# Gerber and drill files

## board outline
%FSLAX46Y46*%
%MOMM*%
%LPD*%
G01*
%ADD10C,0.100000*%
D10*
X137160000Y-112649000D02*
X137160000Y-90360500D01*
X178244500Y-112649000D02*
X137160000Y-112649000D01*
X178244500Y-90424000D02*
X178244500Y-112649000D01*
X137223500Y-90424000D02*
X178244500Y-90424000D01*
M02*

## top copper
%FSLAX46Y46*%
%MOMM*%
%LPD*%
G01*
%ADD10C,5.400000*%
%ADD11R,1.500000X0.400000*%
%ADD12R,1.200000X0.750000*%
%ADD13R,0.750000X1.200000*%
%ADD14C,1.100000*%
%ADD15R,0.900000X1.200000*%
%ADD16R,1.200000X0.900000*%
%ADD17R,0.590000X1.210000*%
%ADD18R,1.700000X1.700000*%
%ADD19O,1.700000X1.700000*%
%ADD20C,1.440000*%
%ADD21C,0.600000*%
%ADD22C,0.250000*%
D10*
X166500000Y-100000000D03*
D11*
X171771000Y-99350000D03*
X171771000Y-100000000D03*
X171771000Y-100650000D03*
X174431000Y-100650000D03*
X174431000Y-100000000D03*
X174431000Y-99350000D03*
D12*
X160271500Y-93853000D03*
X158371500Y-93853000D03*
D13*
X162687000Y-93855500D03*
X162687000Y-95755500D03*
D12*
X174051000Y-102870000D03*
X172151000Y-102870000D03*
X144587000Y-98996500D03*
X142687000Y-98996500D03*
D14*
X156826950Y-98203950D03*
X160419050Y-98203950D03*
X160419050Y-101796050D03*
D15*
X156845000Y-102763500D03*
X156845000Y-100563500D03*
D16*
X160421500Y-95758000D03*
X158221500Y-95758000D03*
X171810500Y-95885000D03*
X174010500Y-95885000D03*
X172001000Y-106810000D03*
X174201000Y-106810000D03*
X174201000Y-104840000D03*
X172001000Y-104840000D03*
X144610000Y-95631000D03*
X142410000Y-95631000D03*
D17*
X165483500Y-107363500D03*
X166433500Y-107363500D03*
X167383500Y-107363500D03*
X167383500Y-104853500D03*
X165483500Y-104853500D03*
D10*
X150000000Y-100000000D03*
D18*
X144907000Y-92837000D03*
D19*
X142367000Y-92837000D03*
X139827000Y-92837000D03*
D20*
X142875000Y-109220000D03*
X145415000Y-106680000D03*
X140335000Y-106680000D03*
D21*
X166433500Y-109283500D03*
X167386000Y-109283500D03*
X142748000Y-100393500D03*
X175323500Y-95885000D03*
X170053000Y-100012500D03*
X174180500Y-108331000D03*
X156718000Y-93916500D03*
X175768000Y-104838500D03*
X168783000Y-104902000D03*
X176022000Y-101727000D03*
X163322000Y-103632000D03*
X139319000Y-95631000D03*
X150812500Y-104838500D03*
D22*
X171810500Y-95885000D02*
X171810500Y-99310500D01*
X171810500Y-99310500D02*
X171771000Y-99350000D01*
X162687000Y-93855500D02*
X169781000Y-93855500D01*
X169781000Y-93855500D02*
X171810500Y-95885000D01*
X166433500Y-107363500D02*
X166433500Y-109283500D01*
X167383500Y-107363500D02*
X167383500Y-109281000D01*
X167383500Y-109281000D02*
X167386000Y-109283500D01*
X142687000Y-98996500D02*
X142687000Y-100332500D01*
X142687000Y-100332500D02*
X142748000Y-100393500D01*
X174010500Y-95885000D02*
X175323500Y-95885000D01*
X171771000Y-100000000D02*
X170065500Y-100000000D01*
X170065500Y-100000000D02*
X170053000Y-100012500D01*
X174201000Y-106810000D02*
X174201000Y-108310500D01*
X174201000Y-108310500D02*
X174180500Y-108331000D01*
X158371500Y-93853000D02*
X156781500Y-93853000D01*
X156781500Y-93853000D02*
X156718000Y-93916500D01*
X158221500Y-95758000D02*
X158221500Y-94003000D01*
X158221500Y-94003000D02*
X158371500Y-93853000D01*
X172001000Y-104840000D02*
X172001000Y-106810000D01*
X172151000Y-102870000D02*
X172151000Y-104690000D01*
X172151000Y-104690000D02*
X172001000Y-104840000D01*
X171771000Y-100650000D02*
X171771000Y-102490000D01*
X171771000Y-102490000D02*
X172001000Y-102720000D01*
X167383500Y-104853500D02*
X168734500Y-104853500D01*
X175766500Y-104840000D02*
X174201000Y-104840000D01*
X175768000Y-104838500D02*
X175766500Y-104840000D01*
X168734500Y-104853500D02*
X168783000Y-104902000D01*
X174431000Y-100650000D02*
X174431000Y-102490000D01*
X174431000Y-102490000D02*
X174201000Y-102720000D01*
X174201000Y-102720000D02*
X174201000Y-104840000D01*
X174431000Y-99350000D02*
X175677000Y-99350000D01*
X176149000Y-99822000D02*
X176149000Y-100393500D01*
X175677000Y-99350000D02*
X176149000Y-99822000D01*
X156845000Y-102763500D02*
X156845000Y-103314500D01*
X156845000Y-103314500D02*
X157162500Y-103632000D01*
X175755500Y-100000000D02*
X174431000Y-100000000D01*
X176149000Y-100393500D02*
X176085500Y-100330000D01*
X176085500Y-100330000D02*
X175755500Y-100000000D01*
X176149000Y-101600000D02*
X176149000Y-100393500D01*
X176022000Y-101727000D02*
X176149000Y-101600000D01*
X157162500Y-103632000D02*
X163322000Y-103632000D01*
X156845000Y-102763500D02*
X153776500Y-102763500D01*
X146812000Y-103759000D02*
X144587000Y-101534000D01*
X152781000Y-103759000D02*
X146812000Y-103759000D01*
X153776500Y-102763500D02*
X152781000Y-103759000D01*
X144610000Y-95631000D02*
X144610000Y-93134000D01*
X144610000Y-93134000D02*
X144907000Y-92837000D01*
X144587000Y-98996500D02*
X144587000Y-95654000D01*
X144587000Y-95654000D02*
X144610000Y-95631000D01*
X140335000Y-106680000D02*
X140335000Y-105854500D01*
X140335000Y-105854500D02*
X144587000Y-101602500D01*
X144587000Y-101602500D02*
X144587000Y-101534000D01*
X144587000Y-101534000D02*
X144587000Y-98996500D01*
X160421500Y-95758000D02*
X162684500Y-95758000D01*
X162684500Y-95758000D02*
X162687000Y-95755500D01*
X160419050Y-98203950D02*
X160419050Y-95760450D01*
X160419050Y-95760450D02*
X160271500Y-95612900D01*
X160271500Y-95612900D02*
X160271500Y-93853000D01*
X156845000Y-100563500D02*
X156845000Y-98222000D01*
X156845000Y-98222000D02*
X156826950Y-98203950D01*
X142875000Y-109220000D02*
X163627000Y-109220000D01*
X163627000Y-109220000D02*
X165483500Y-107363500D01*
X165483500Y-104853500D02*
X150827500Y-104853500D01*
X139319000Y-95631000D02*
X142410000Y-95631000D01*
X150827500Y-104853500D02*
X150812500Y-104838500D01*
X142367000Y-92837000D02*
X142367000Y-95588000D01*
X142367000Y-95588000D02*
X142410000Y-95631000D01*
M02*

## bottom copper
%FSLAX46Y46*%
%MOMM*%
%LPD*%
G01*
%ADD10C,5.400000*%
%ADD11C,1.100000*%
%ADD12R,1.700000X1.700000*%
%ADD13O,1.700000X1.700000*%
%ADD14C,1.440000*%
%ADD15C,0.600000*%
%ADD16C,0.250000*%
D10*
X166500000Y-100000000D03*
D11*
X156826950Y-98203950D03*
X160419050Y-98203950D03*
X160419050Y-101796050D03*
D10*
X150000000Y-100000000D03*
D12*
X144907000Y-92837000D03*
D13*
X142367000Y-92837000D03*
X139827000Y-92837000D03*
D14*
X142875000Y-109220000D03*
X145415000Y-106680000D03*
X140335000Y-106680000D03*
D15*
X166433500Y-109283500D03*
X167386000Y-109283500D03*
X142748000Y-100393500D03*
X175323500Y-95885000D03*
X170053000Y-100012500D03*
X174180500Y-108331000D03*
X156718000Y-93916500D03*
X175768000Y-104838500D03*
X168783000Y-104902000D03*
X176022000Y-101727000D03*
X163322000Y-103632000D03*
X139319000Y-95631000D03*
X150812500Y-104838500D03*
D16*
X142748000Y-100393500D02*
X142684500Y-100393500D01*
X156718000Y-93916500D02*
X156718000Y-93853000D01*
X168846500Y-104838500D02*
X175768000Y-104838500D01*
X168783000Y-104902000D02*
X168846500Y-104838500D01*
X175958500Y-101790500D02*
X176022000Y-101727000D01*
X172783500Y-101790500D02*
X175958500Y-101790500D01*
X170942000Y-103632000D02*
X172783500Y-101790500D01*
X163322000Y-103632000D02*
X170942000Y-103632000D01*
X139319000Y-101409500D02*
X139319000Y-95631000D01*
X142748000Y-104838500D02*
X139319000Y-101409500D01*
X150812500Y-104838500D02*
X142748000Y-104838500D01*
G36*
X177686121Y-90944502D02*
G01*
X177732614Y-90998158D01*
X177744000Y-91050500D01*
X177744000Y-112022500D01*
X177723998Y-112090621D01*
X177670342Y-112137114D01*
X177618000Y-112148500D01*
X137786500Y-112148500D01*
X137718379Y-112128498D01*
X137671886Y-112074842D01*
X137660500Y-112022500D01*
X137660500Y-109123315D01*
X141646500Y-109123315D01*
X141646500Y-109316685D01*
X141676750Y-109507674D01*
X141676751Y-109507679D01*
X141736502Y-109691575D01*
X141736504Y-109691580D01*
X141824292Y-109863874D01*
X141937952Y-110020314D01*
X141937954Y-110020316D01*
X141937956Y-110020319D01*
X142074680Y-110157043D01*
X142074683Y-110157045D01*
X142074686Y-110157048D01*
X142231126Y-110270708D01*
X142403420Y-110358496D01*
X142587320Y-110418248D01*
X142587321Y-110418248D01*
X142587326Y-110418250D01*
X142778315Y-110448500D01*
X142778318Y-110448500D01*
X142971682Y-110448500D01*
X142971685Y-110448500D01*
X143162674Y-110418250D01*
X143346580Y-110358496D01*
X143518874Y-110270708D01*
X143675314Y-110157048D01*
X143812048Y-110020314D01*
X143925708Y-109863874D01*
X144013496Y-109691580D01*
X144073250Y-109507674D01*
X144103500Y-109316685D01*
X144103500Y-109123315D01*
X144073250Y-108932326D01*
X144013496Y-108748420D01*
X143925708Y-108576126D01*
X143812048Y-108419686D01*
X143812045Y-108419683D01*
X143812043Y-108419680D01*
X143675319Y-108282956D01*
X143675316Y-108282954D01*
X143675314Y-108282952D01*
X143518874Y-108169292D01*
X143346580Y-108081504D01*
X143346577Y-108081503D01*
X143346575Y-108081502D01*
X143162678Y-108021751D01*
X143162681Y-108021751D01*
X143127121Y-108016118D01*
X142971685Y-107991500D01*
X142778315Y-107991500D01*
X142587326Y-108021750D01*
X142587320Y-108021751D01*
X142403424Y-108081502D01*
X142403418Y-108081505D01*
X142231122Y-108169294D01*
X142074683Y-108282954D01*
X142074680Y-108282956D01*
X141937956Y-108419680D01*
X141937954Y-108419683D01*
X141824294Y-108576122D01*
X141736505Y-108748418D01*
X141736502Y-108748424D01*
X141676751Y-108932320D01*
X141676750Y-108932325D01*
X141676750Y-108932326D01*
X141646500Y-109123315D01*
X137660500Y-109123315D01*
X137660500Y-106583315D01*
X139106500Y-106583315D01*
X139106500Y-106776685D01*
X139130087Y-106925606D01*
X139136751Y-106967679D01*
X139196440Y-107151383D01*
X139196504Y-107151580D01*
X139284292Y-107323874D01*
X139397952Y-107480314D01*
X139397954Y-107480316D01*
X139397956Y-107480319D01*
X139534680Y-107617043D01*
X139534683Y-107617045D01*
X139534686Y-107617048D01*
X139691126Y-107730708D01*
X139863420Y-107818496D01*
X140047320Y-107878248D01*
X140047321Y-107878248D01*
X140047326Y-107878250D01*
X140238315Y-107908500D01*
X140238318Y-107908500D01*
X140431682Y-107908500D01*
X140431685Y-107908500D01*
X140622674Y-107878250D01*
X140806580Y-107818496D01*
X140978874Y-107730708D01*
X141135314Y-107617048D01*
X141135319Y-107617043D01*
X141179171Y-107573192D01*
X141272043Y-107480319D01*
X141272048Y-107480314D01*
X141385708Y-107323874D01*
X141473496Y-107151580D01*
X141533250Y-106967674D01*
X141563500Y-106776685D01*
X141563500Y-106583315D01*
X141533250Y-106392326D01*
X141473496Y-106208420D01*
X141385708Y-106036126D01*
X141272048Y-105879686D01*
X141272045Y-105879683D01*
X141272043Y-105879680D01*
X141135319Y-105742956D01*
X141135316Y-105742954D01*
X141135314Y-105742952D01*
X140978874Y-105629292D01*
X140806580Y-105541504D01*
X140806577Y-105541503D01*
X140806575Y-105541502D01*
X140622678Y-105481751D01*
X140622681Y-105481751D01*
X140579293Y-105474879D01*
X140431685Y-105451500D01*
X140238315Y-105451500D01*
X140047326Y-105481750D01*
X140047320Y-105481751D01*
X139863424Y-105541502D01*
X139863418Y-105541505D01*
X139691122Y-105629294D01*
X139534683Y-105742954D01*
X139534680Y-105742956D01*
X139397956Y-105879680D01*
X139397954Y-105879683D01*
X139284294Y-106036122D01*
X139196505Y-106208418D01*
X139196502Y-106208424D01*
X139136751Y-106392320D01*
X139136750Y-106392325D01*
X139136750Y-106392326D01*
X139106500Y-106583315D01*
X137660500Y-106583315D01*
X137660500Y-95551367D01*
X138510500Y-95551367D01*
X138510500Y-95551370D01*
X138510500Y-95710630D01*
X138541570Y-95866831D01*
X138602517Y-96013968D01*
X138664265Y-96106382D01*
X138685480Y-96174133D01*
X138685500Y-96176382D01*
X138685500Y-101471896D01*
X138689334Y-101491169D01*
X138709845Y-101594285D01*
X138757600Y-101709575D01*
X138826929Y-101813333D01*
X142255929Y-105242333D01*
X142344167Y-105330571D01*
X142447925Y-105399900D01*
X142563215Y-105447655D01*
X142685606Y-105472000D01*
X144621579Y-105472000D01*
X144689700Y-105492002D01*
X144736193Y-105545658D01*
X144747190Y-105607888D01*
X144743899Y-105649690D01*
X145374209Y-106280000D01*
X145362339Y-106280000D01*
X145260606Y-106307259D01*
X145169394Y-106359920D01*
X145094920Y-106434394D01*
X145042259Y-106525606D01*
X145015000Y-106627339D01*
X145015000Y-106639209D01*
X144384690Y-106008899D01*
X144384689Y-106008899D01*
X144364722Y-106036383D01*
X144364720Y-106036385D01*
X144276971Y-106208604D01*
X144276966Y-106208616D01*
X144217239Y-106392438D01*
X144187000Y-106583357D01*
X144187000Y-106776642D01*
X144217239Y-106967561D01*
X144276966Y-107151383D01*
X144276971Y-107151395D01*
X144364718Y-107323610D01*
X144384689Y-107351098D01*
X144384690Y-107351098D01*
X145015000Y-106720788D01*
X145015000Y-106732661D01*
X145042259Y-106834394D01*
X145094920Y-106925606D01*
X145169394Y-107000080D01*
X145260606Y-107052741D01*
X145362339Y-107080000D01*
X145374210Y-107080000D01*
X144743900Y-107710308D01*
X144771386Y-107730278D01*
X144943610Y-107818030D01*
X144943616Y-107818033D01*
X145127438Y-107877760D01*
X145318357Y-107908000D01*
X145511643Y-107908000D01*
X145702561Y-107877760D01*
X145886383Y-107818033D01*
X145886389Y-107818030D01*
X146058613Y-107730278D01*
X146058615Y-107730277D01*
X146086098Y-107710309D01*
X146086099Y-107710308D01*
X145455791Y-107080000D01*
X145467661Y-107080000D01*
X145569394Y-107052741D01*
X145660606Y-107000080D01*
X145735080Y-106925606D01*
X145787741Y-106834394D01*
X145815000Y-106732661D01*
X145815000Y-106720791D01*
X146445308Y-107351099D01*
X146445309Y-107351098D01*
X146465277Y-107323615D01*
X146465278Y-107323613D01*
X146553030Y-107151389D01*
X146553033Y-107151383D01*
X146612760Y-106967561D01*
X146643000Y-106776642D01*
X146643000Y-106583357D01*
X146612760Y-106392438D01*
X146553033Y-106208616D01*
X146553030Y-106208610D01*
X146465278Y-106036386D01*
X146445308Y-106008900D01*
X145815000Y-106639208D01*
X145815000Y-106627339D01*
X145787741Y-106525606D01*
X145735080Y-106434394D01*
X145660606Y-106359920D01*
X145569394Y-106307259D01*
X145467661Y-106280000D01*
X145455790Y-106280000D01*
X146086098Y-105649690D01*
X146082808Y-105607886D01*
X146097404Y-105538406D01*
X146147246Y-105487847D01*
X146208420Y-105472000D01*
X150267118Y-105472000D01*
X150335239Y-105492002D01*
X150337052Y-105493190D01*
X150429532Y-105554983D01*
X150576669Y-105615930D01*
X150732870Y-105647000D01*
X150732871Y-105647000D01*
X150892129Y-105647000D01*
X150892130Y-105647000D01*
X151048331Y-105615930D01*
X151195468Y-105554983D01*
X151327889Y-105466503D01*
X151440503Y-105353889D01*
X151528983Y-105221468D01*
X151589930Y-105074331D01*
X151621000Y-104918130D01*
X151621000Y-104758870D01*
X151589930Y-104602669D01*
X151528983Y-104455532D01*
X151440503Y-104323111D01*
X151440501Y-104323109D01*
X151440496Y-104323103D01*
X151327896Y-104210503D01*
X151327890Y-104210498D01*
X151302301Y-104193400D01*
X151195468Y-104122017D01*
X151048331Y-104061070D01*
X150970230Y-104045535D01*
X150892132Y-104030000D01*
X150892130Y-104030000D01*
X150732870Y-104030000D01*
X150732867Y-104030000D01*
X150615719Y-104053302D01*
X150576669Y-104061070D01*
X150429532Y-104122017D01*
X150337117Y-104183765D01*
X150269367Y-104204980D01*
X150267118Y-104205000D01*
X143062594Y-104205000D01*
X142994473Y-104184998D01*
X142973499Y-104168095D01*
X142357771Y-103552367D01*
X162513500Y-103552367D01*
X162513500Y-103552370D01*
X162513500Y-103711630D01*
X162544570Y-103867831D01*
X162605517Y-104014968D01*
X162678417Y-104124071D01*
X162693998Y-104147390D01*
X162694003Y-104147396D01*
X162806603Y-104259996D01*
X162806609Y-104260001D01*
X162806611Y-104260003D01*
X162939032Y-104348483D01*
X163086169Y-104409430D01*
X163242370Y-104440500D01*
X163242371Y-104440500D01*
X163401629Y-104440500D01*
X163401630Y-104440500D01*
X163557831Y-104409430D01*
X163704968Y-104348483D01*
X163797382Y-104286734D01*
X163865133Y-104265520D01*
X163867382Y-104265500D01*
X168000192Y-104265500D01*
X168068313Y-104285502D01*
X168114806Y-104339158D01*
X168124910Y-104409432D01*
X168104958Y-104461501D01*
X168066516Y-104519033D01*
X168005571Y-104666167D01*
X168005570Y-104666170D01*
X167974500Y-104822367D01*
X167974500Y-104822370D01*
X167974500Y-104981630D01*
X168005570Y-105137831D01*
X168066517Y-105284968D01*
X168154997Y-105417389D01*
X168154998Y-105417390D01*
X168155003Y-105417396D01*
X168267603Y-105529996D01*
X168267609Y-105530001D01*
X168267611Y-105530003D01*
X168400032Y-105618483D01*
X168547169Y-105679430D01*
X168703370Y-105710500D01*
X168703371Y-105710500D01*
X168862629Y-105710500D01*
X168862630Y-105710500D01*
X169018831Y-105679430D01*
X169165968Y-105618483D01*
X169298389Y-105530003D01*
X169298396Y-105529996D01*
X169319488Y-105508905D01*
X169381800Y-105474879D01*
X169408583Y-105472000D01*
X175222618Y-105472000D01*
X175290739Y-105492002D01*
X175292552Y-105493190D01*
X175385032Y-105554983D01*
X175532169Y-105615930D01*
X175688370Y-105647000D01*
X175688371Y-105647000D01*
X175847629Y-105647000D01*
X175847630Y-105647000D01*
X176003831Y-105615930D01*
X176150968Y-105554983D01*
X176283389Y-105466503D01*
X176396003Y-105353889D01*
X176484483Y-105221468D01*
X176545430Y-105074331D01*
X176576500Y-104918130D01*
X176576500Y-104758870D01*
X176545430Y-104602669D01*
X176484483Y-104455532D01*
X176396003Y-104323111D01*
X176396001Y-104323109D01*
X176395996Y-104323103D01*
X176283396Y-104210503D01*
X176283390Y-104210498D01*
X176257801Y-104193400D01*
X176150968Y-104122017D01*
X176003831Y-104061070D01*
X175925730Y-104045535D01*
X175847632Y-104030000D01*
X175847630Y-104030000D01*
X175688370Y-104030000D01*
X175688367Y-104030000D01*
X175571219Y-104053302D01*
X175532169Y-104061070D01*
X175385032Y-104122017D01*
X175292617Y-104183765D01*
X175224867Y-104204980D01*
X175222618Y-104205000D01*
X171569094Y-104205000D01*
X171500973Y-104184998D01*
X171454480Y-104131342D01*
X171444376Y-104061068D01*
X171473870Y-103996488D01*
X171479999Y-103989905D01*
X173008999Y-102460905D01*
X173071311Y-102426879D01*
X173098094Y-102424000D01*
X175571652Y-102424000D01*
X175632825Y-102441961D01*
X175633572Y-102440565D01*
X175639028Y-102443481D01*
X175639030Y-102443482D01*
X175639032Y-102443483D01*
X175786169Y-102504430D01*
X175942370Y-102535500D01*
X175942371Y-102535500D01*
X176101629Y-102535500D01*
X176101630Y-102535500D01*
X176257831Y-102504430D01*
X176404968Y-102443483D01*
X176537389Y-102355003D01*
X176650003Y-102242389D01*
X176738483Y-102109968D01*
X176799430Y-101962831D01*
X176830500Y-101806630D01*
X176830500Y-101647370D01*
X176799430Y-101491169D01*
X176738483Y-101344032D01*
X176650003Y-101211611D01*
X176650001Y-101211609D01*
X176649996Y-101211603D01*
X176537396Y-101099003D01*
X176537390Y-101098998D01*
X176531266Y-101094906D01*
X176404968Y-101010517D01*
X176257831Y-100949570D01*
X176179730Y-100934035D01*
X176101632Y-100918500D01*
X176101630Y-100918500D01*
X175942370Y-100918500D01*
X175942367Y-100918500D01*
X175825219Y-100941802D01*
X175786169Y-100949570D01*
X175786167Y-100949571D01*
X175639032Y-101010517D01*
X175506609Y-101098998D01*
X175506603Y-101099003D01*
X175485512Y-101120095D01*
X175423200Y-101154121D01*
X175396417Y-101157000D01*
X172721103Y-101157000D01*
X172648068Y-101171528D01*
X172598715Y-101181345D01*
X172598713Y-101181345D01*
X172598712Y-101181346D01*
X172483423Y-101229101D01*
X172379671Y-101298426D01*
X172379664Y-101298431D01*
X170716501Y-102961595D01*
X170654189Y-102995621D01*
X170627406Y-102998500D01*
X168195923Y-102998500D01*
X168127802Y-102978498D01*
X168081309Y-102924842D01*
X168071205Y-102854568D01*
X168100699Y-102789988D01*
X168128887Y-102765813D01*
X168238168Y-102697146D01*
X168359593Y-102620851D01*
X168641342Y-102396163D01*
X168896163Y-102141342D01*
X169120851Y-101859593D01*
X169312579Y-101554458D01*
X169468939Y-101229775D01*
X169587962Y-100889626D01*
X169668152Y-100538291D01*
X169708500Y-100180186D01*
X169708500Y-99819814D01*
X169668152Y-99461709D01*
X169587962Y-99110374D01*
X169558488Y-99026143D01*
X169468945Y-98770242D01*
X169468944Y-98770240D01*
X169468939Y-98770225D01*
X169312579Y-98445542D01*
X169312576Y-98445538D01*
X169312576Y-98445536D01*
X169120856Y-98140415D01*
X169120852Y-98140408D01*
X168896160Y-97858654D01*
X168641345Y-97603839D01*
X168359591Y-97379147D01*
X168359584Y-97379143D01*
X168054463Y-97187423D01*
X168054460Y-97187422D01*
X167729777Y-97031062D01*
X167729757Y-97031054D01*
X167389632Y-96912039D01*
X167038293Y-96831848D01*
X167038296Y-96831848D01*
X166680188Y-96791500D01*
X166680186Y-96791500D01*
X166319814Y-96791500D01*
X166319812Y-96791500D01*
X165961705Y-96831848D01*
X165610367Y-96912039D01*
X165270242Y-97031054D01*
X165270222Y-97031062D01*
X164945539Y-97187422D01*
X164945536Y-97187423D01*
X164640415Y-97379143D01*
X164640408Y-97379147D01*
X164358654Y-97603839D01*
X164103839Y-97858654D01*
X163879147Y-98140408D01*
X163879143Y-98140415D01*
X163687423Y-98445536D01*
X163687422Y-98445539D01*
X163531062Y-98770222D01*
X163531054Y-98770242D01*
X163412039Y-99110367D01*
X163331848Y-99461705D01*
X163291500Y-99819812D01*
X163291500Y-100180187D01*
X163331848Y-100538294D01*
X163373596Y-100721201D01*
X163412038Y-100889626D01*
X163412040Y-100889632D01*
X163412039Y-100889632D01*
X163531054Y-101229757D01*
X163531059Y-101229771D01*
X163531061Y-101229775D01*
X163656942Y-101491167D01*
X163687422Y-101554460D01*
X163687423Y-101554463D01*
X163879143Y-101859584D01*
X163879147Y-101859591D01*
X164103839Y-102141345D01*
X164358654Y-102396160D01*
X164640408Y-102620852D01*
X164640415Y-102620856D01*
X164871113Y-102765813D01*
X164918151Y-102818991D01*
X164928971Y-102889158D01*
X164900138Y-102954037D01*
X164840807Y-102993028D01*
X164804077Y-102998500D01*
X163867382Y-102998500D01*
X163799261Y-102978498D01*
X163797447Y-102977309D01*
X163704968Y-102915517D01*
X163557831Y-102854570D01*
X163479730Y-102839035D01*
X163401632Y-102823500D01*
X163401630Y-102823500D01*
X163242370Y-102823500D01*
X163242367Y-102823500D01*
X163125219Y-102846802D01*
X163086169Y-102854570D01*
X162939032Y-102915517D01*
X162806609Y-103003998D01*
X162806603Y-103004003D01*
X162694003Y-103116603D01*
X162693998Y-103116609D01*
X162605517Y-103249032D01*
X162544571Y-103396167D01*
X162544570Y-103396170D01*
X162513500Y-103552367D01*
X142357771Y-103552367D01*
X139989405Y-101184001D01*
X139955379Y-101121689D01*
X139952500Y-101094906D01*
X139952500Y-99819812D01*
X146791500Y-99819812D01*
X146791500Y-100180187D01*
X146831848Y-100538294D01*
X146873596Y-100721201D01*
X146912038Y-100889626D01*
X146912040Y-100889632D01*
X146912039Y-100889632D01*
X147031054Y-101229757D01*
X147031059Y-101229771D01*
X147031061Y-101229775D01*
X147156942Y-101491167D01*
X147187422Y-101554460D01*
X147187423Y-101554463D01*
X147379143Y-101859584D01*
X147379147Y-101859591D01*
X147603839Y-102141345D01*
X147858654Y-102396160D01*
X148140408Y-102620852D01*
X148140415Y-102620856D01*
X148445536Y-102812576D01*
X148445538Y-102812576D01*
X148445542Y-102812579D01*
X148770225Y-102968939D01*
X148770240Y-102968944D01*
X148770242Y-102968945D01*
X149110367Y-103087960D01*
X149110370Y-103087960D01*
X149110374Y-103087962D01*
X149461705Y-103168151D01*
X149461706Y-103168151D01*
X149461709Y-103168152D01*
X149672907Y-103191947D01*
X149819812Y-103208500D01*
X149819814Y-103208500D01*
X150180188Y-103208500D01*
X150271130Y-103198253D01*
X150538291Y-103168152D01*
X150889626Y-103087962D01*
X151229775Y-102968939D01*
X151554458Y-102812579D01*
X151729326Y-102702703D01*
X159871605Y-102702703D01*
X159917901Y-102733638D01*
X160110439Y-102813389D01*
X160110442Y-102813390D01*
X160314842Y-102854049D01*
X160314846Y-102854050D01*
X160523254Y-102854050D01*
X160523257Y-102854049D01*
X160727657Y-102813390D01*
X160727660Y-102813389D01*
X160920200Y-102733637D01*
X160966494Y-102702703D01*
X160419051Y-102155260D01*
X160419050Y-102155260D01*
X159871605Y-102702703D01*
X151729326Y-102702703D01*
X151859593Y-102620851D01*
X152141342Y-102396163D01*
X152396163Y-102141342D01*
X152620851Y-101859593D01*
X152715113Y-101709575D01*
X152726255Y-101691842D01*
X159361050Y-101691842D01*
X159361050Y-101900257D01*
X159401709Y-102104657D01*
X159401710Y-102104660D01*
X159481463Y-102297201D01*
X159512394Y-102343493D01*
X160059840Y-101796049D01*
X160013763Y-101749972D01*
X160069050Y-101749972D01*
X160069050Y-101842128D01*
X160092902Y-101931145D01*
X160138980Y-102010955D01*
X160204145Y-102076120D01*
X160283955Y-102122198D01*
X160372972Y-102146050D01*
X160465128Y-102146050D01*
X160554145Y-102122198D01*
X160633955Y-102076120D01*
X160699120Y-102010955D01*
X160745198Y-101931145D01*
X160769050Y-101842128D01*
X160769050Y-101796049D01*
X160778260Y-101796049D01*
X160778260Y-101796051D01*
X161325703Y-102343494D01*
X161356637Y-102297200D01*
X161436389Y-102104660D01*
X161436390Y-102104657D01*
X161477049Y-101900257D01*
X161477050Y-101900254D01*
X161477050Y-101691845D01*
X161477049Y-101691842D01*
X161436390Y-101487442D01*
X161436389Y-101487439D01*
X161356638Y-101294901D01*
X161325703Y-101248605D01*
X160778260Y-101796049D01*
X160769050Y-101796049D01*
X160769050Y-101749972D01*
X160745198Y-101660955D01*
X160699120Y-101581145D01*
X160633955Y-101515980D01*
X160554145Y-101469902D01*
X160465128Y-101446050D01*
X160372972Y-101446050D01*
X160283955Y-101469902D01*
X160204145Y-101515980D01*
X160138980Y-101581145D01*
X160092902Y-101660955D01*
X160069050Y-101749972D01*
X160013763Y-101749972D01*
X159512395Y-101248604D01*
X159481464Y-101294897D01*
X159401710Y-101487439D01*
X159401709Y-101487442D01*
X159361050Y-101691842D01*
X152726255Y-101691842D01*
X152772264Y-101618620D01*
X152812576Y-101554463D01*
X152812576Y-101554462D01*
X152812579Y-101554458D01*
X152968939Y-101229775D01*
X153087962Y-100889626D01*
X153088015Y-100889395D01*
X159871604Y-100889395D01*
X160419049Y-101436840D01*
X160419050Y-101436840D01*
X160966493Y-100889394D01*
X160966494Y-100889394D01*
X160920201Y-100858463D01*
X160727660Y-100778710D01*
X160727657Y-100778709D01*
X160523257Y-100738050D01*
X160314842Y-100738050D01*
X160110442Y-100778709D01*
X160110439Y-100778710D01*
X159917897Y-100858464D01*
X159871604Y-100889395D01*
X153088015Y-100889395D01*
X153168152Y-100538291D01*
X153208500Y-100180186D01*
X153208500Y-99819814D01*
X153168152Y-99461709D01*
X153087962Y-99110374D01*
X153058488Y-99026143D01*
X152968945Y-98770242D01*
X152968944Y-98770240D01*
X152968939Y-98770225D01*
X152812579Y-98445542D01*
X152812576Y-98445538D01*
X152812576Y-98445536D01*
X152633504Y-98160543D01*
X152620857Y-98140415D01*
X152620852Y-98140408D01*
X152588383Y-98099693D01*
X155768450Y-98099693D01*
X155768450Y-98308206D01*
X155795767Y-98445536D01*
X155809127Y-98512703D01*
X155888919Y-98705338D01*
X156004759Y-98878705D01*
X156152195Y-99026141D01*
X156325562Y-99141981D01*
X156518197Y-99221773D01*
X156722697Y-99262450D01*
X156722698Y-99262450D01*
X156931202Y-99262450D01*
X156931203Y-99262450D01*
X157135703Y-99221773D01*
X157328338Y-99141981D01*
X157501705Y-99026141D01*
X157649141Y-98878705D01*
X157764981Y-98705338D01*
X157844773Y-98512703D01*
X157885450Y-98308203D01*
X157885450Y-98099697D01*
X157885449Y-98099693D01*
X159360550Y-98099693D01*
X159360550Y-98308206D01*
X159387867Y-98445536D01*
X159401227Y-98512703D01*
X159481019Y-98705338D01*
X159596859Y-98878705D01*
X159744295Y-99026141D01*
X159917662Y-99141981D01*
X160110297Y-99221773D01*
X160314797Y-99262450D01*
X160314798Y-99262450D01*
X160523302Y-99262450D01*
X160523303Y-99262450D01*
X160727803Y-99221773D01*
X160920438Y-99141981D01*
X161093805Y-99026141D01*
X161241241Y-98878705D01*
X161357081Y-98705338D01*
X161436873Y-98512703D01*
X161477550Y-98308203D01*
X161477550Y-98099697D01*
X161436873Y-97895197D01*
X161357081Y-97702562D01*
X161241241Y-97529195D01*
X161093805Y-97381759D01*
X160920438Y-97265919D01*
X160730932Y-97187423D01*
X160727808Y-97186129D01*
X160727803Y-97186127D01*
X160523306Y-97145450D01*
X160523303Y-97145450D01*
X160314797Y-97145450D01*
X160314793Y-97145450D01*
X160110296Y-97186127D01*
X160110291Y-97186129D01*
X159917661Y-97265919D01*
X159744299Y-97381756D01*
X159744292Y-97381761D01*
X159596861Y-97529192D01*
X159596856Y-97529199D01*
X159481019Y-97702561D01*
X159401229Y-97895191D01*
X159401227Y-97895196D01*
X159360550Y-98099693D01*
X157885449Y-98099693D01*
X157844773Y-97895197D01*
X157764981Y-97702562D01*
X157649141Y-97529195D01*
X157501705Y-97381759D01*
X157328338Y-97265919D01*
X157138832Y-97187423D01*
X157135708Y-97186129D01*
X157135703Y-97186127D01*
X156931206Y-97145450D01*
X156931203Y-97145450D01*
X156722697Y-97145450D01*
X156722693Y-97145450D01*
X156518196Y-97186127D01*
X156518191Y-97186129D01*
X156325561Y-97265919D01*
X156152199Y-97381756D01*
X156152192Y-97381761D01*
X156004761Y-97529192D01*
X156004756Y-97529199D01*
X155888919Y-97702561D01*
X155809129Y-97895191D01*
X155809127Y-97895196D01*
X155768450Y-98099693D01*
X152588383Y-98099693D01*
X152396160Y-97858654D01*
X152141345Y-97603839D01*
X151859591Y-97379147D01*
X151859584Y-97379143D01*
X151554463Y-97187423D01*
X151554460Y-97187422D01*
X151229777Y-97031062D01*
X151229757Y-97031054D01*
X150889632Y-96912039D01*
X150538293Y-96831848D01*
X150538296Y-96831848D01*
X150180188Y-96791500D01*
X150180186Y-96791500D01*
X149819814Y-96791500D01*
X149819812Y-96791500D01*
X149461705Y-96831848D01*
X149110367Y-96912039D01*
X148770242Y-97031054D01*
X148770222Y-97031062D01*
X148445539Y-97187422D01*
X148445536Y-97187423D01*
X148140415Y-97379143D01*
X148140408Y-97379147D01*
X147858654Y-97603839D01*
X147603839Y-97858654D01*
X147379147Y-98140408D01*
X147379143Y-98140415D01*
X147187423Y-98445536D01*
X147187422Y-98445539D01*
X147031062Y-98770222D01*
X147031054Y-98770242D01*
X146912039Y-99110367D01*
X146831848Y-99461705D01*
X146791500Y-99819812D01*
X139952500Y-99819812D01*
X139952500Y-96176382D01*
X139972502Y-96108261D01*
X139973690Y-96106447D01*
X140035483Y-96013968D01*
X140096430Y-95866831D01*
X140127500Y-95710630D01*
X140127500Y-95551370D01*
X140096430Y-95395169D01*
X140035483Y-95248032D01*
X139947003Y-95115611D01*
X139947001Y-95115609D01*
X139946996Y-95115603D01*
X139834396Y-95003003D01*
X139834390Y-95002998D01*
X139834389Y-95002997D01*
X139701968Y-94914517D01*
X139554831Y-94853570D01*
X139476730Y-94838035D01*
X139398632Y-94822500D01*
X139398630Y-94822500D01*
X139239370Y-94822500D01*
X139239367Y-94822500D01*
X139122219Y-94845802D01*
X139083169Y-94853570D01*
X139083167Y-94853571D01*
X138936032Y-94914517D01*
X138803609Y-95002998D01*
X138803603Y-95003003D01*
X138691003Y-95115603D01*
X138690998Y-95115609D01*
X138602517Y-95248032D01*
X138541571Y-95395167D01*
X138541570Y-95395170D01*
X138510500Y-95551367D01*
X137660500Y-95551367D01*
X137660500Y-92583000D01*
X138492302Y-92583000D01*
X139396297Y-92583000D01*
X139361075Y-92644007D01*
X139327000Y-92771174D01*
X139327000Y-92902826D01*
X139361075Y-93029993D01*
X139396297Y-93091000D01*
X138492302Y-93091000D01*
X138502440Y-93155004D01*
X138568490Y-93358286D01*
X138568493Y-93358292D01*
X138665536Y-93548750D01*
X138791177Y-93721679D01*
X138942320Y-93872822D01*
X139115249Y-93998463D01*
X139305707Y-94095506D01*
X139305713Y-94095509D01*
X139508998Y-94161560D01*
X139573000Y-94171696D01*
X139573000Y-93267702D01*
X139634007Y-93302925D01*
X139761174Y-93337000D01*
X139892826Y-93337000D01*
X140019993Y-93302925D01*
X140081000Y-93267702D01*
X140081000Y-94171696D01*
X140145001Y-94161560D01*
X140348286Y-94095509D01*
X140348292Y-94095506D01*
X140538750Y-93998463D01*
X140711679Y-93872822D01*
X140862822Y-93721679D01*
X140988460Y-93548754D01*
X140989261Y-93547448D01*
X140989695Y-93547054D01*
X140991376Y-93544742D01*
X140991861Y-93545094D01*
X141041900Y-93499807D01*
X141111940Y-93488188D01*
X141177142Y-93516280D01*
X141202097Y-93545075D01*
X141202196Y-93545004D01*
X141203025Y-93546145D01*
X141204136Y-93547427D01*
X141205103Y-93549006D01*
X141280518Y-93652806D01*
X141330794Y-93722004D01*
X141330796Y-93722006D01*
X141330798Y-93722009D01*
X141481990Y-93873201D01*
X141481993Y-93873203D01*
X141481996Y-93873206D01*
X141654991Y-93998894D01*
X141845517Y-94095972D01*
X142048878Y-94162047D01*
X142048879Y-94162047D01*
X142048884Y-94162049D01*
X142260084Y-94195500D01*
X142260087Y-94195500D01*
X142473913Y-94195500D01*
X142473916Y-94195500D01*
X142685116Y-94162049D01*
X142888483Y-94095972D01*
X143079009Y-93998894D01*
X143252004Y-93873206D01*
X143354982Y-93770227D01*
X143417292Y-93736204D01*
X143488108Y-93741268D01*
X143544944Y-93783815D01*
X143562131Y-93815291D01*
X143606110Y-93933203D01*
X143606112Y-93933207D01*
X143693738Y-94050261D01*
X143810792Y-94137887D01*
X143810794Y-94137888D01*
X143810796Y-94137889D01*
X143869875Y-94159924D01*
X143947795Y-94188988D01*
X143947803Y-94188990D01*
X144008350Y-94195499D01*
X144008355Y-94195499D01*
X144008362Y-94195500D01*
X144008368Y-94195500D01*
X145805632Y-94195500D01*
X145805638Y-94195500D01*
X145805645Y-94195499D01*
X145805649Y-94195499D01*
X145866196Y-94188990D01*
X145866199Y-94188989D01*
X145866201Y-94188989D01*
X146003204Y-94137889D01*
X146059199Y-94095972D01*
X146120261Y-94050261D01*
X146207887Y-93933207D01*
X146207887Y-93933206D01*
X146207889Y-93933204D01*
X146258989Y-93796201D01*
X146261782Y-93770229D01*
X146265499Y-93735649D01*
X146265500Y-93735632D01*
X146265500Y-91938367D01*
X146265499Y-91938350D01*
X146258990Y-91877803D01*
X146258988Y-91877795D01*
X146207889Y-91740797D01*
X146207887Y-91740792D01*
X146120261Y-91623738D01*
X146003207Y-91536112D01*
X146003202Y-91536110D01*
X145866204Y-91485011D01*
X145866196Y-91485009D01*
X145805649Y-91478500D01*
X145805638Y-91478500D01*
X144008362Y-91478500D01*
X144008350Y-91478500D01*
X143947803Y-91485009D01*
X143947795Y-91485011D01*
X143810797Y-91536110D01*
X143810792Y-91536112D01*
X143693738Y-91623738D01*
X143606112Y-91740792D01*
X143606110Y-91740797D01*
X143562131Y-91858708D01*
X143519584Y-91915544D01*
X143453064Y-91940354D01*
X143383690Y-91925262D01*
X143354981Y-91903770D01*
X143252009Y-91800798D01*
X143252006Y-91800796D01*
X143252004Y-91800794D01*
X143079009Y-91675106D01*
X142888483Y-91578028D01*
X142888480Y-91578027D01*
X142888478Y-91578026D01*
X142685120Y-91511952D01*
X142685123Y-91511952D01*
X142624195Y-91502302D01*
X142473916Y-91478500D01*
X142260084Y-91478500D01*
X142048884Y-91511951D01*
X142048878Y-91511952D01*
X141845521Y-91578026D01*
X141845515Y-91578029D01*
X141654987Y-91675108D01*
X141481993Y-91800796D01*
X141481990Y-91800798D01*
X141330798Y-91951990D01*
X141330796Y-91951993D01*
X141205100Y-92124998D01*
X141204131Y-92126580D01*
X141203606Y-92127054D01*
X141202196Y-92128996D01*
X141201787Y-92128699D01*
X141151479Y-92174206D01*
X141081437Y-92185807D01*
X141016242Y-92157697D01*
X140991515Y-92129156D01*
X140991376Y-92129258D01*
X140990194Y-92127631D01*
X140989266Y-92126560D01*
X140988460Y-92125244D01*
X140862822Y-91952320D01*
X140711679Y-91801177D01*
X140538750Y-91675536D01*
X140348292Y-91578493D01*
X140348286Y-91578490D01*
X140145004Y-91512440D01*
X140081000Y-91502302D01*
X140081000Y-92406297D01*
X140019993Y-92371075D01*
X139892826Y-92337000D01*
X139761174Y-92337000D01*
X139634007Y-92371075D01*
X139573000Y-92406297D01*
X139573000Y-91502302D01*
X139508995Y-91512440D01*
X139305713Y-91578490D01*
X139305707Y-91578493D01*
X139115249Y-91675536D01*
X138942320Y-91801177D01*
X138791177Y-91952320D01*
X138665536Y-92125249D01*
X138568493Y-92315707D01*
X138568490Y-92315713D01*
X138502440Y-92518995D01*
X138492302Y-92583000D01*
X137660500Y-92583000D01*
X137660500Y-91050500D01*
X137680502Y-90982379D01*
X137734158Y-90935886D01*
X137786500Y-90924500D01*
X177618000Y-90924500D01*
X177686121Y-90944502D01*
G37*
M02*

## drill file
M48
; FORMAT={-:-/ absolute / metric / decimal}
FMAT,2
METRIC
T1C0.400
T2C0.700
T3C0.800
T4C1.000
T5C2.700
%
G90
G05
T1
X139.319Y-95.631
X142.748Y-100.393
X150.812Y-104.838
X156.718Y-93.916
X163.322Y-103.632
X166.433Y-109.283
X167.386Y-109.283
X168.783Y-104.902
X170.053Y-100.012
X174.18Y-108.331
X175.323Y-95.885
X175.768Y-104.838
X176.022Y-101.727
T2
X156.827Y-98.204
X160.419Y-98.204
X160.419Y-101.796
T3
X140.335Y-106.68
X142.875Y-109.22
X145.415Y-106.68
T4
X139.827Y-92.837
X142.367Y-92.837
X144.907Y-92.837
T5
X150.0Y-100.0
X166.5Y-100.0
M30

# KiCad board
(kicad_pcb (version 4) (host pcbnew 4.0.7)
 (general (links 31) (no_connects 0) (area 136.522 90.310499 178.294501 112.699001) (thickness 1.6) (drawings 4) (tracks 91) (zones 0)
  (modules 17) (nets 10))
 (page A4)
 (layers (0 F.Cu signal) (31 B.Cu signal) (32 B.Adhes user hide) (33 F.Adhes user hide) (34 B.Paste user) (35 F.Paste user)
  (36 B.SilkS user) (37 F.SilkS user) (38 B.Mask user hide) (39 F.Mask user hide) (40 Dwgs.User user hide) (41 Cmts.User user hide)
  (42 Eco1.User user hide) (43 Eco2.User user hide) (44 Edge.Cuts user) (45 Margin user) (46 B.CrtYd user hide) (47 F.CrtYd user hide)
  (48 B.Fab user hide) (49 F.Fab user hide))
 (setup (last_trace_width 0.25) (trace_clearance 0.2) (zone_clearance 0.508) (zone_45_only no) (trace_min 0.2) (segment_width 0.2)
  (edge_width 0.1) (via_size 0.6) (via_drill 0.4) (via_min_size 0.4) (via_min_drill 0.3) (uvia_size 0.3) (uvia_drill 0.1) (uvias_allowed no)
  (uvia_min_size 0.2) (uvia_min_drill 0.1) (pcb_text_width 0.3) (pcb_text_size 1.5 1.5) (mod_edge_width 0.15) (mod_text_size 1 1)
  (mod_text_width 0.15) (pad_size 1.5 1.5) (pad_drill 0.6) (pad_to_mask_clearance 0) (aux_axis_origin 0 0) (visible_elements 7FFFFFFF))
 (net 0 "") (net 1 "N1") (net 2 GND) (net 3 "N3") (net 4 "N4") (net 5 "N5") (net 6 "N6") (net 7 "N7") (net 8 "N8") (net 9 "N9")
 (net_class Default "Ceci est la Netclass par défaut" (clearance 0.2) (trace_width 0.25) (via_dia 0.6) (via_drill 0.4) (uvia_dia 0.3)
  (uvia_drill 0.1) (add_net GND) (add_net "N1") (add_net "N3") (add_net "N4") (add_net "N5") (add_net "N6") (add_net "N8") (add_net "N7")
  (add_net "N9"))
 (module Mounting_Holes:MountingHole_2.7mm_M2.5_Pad (layer F.Cu) (at 166.5 100)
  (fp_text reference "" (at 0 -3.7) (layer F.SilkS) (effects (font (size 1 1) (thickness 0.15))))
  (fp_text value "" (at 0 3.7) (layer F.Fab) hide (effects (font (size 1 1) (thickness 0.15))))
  (pad 1 thru_hole circle (at 0 0) (size 5.4 5.4) (drill 2.7) (layers *.Cu *.Mask)))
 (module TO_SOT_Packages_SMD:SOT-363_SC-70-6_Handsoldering (layer F.Cu) (at 173.101 100)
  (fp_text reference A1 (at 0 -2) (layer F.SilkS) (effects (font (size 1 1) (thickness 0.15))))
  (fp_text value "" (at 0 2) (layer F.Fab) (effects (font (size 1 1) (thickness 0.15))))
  (pad 1 smd rect (at -1.33 -0.65) (size 1.5 0.4) (layers F.Cu F.Paste F.Mask) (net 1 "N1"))
  (pad 2 smd rect (at -1.33 0) (size 1.5 0.4) (layers F.Cu F.Paste F.Mask) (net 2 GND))
  (pad 3 smd rect (at -1.33 0.65) (size 1.5 0.4) (layers F.Cu F.Paste F.Mask) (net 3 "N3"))
  (pad 4 smd rect (at 1.33 0.65) (size 1.5 0.4) (layers F.Cu F.Paste F.Mask) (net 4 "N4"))
  (pad 5 smd rect (at 1.33 0) (size 1.5 0.4) (layers F.Cu F.Paste F.Mask) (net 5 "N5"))
  (pad 6 smd rect (at 1.33 -0.65) (size 1.5 0.4) (layers F.Cu F.Paste F.Mask) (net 5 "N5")))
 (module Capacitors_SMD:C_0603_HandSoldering (layer F.Cu) (at 159.3215 93.853 180)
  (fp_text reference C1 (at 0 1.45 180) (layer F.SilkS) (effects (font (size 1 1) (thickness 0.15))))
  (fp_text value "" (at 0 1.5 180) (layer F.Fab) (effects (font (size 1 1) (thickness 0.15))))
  (pad 1 smd rect (at -0.95 0 180) (size 1.2 0.75) (layers F.Cu F.Paste F.Mask) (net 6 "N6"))
  (pad 2 smd rect (at 0.95 0 180) (size 1.2 0.75) (layers F.Cu F.Paste F.Mask) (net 2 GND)))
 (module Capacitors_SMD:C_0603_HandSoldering (layer F.Cu) (at 162.687 94.8055 270)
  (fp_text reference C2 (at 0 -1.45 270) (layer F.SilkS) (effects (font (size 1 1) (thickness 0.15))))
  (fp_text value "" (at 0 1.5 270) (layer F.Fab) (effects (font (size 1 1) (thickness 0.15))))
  (pad 1 smd rect (at -0.95 0 270) (size 1.2 0.75) (layers F.Cu F.Paste F.Mask) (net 1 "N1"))
  (pad 2 smd rect (at 0.95 0 270) (size 1.2 0.75) (layers F.Cu F.Paste F.Mask) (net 6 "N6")))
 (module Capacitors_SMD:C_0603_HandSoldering (layer F.Cu) (at 173.101 102.87 180)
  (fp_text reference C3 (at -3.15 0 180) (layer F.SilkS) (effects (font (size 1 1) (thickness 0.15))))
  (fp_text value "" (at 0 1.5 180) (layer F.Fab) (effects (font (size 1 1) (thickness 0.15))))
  (pad 1 smd rect (at -0.95 0 180) (size 1.2 0.75) (layers F.Cu F.Paste F.Mask) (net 4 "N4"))
  (pad 2 smd rect (at 0.95 0 180) (size 1.2 0.75) (layers F.Cu F.Paste F.Mask) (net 3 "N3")))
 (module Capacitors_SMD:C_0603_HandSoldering (layer F.Cu) (at 143.637 98.9965 180)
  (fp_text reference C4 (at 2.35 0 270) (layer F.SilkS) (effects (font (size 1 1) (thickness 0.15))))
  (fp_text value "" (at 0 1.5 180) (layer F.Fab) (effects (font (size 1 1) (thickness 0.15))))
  (pad 1 smd rect (at -0.95 0 180) (size 1.2 0.75) (layers F.Cu F.Paste F.Mask) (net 5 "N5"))
  (pad 2 smd rect (at 0.95 0 180) (size 1.2 0.75) (layers F.Cu F.Paste F.Mask) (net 2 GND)))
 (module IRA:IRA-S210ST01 (layer B.Cu) (at 158.623 100)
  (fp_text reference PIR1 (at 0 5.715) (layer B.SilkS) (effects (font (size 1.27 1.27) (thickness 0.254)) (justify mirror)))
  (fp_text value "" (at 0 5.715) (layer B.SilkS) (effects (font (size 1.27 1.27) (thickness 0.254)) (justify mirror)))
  (pad 1 thru_hole circle (at -1.79605 -1.79605 270) (size 1.1 1.1) (drill 0.7) (layers *.Cu *.Mask B.SilkS) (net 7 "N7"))
  (pad 2 thru_hole circle (at 1.79605 -1.79605 270) (size 1.1 1.1) (drill 0.7) (layers *.Cu *.Mask B.SilkS) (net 6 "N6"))
  (pad 3 thru_hole circle (at 1.79605 1.79605 270) (size 1.1 1.1) (drill 0.7) (layers *.Cu *.Mask B.SilkS) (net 2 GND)))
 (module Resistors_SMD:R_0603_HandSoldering (layer F.Cu) (at 156.845 101.6635 90)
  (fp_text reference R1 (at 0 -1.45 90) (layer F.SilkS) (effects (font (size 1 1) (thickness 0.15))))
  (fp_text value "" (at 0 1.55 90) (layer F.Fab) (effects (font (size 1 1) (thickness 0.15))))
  (pad 1 smd rect (at -1.1 0 90) (size 1.2 0.9) (layers F.Cu F.Paste F.Mask) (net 5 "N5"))
  (pad 2 smd rect (at 1.1 0 90) (size 1.2 0.9) (layers F.Cu F.Paste F.Mask) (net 7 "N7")))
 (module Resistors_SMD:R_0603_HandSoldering (layer F.Cu) (at 159.3215 95.758 180)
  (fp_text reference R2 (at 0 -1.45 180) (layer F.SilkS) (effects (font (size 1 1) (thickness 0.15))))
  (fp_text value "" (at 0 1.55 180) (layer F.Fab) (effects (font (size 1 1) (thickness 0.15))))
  (pad 1 smd rect (at -1.1 0 180) (size 1.2 0.9) (layers F.Cu F.Paste F.Mask) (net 6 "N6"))
  (pad 2 smd rect (at 1.1 0 180) (size 1.2 0.9) (layers F.Cu F.Paste F.Mask) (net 2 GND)))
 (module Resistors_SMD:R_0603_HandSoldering (layer F.Cu) (at 172.9105 95.885)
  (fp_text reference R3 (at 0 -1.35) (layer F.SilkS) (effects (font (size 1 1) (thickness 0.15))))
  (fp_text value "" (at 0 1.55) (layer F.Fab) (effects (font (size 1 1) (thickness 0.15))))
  (pad 1 smd rect (at -1.1 0) (size 1.2 0.9) (layers F.Cu F.Paste F.Mask) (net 1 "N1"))
  (pad 2 smd rect (at 1.1 0) (size 1.2 0.9) (layers F.Cu F.Paste F.Mask) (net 2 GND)))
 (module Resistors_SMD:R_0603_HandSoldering (layer F.Cu) (at 173.101 106.81)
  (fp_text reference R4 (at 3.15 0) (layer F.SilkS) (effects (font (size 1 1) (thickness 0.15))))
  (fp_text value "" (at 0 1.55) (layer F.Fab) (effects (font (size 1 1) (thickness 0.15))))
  (pad 1 smd rect (at -1.1 0) (size 1.2 0.9) (layers F.Cu F.Paste F.Mask) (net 3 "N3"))
  (pad 2 smd rect (at 1.1 0) (size 1.2 0.9) (layers F.Cu F.Paste F.Mask) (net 2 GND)))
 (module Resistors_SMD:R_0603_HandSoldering (layer F.Cu) (at 173.101 104.84 180)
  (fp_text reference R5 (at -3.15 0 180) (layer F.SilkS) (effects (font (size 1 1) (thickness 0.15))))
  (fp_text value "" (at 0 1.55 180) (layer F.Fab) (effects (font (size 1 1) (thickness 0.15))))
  (pad 1 smd rect (at -1.1 0 180) (size 1.2 0.9) (layers F.Cu F.Paste F.Mask) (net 4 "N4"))
  (pad 2 smd rect (at 1.1 0 180) (size 1.2 0.9) (layers F.Cu F.Paste F.Mask) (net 3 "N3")))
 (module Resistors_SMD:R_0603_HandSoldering (layer F.Cu) (at 143.51 95.631 180)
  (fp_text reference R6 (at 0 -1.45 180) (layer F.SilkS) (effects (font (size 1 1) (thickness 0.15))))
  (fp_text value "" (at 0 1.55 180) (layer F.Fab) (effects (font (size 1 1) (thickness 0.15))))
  (pad 1 smd rect (at -1.1 0 180) (size 1.2 0.9) (layers F.Cu F.Paste F.Mask) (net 5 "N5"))
  (pad 2 smd rect (at 1.1 0 180) (size 1.2 0.9) (layers F.Cu F.Paste F.Mask) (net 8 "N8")))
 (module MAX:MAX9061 (layer F.Cu) (at 166.4335 106.1085 90)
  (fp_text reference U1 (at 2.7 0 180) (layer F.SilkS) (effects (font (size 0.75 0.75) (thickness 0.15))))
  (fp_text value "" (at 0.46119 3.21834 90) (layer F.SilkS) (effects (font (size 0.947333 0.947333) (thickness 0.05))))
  (pad 1 smd rect (at -1.255 -0.95 270) (size 1.21 0.59) (layers F.Cu F.Paste F.Mask) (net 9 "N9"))
  (pad 2 smd rect (at -1.255 0 270) (size 1.21 0.59) (layers F.Cu F.Paste F.Mask) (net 2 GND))
  (pad 3 smd rect (at -1.255 0.95 270) (size 1.21 0.59) (layers F.Cu F.Paste F.Mask) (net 2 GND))
  (pad 4 smd rect (at 1.255 0.95 90) (size 1.21 0.59) (layers F.Cu F.Paste F.Mask) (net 4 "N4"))
  (pad 5 smd rect (at 1.255 -0.95 90) (size 1.21 0.59) (layers F.Cu F.Paste F.Mask) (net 8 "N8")))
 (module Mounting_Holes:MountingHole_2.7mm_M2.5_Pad (layer F.Cu) (at 150 100)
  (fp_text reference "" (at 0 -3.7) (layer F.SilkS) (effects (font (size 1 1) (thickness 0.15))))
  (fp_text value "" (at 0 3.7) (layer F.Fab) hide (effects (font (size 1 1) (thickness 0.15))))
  (pad 1 thru_hole circle (at 0 0) (size 5.4 5.4) (drill 2.7) (layers *.Cu *.Mask)))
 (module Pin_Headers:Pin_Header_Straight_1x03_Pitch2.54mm (layer F.Cu) (at 144.907 92.837 270)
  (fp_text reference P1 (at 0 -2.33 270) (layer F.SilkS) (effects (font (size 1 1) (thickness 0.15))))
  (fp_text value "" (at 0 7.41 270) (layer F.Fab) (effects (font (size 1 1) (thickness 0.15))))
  (pad 1 thru_hole rect (at 0 0 270) (size 1.7 1.7) (drill 1) (layers *.Cu *.Mask) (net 5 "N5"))
  (pad 2 thru_hole oval (at 0 2.54 270) (size 1.7 1.7) (drill 1) (layers *.Cu *.Mask) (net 8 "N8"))
  (pad 3 thru_hole oval (at 0 5.08 270) (size 1.7 1.7) (drill 1) (layers *.Cu *.Mask) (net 2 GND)))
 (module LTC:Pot (layer F.Cu) (at 140.335 106.68)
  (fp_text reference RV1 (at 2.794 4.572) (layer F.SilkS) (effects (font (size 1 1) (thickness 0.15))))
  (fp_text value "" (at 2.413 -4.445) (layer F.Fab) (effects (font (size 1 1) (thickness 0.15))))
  (pad 2 thru_hole circle (at 2.54 2.54) (size 1.44 1.44) (drill 0.8) (layers *.Cu *.Mask) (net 9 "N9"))
  (pad 3 thru_hole circle (at 5.08 0) (size 1.44 1.44) (drill 0.8) (layers *.Cu *.Mask) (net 2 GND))
  (pad 1 thru_hole circle (at 0 0) (size 1.44 1.44) (drill 0.8) (layers *.Cu *.Mask) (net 5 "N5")))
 (gr_line (start 137.16 112.649) (end 137.16 90.3605) (angle 90) (layer Edge.Cuts) (width 0.1))
 (gr_line (start 178.2445 112.649) (end 137.16 112.649) (angle 90) (layer Edge.Cuts) (width 0.1))
 (gr_line (start 178.2445 90.424) (end 178.2445 112.649) (angle 90) (layer Edge.Cuts) (width 0.1))
 (gr_line (start 137.2235 90.424) (end 178.2445 90.424) (angle 90) (layer Edge.Cuts) (width 0.1))
 (segment (start 171.8105 95.885) (end 171.8105 99.3105) (width 0.25) (layer F.Cu) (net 1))
 (segment (start 171.8105 99.3105) (end 171.771 99.35) (width 0.25) (layer F.Cu) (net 1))
 (segment (start 162.687 93.8555) (end 169.781 93.8555) (width 0.25) (layer F.Cu) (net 1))
 (segment (start 169.781 93.8555) (end 171.8105 95.885) (width 0.25) (layer F.Cu) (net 1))
 (segment (start 166.4335 107.3635) (end 166.4335 109.2835) (width 0.25) (layer F.Cu) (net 2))
 (via (at 166.4335 109.2835) (size 0.6) (drill 0.4) (layers F.Cu B.Cu) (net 2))
 (segment (start 167.3835 107.3635) (end 167.3835 109.281) (width 0.25) (layer F.Cu) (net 2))
 (via (at 167.386 109.2835) (size 0.6) (drill 0.4) (layers F.Cu B.Cu) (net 2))
 (segment (start 167.3835 109.281) (end 167.386 109.2835) (width 0.25) (layer F.Cu) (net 2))
 (segment (start 142.687 98.9965) (end 142.687 100.3325) (width 0.25) (layer F.Cu) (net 2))
 (segment (start 142.748 100.3935) (end 142.6845 100.3935) (width 0.25) (layer B.Cu) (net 2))
 (via (at 142.748 100.3935) (size 0.6) (drill 0.4) (layers F.Cu B.Cu) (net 2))
 (segment (start 142.687 100.3325) (end 142.748 100.3935) (width 0.25) (layer F.Cu) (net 2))
 (segment (start 174.0105 95.885) (end 175.3235 95.885) (width 0.25) (layer F.Cu) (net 2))
 (via (at 175.3235 95.885) (size 0.6) (drill 0.4) (layers F.Cu B.Cu) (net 2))
 (segment (start 171.771 100) (end 170.0655 100) (width 0.25) (layer F.Cu) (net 2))
 (via (at 170.053 100.0125) (size 0.6) (drill 0.4) (layers F.Cu B.Cu) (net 2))
 (segment (start 170.0655 100) (end 170.053 100.0125) (width 0.25) (layer F.Cu) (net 2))
 (segment (start 174.201 106.81) (end 174.201 108.3105) (width 0.25) (layer F.Cu) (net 2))
 (via (at 174.1805 108.331) (size 0.6) (drill 0.4) (layers F.Cu B.Cu) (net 2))
 (segment (start 174.201 108.3105) (end 174.1805 108.331) (width 0.25) (layer F.Cu) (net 2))
 (segment (start 158.3715 93.853) (end 156.7815 93.853) (width 0.25) (layer F.Cu) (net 2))
 (segment (start 156.718 93.9165) (end 156.718 93.853) (width 0.25) (layer B.Cu) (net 2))
 (via (at 156.718 93.9165) (size 0.6) (drill 0.4) (layers F.Cu B.Cu) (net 2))
 (segment (start 156.7815 93.853) (end 156.718 93.9165) (width 0.25) (layer F.Cu) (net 2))
 (segment (start 158.2215 95.758) (end 158.2215 94.003) (width 0.25) (layer F.Cu) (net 2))
 (segment (start 158.2215 94.003) (end 158.3715 93.853) (width 0.25) (layer F.Cu) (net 2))
 (segment (start 172.001 104.84) (end 172.001 106.81) (width 0.25) (layer F.Cu) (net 3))
 (segment (start 172.151 102.87) (end 172.151 104.69) (width 0.25) (layer F.Cu) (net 3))
 (segment (start 172.151 104.69) (end 172.001 104.84) (width 0.25) (layer F.Cu) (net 3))
 (segment (start 171.771 100.65) (end 171.771 102.49) (width 0.25) (layer F.Cu) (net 3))
 (segment (start 171.771 102.49) (end 172.001 102.72) (width 0.25) (layer F.Cu) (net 3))
 (segment (start 167.3835 104.8535) (end 168.7345 104.8535) (width 0.25) (layer F.Cu) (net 4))
 (segment (start 175.7665 104.84) (end 174.201 104.84) (width 0.25) (layer F.Cu) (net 4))
 (segment (start 175.768 104.8385) (end 175.7665 104.84) (width 0.25) (layer F.Cu) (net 4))
 (via (at 175.768 104.8385) (size 0.6) (drill 0.4) (layers F.Cu B.Cu) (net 4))
 (segment (start 168.8465 104.8385) (end 175.768 104.8385) (width 0.25) (layer B.Cu) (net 4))
 (segment (start 168.783 104.902) (end 168.8465 104.8385) (width 0.25) (layer B.Cu) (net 4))
 (via (at 168.783 104.902) (size 0.6) (drill 0.4) (layers F.Cu B.Cu) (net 4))
 (segment (start 168.7345 104.8535) (end 168.783 104.902) (width 0.25) (layer F.Cu) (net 4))
 (segment (start 174.431 100.65) (end 174.431 102.49) (width 0.25) (layer F.Cu) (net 4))
 (segment (start 174.431 102.49) (end 174.201 102.72) (width 0.25) (layer F.Cu) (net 4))
 (segment (start 174.201 102.72) (end 174.201 104.84) (width 0.25) (layer F.Cu) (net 4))
 (segment (start 174.431 99.35) (end 175.677 99.35) (width 0.25) (layer F.Cu) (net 5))
 (segment (start 176.149 99.822) (end 176.149 100.3935) (width 0.25) (layer F.Cu) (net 5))
 (segment (start 175.677 99.35) (end 176.149 99.822) (width 0.25) (layer F.Cu) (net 5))
 (segment (start 156.845 102.7635) (end 156.845 103.3145) (width 0.25) (layer F.Cu) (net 5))
 (segment (start 156.845 103.3145) (end 157.1625 103.632) (width 0.25) (layer F.Cu) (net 5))
 (segment (start 175.7555 100) (end 174.431 100) (width 0.25) (layer F.Cu) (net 5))
 (segment (start 176.149 100.3935) (end 176.0855 100.33) (width 0.25) (layer F.Cu) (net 5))
 (segment (start 176.0855 100.33) (end 175.7555 100) (width 0.25) (layer F.Cu) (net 5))
 (segment (start 176.149 101.6) (end 176.149 100.3935) (width 0.25) (layer F.Cu) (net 5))
 (segment (start 176.022 101.727) (end 176.149 101.6) (width 0.25) (layer F.Cu) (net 5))
 (via (at 176.022 101.727) (size 0.6) (drill 0.4) (layers F.Cu B.Cu) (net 5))
 (segment (start 175.9585 101.7905) (end 176.022 101.727) (width 0.25) (layer B.Cu) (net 5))
 (segment (start 172.7835 101.7905) (end 175.9585 101.7905) (width 0.25) (layer B.Cu) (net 5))
 (segment (start 170.942 103.632) (end 172.7835 101.7905) (width 0.25) (layer B.Cu) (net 5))
 (segment (start 163.322 103.632) (end 170.942 103.632) (width 0.25) (layer B.Cu) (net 5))
 (via (at 163.322 103.632) (size 0.6) (drill 0.4) (layers F.Cu B.Cu) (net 5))
 (segment (start 157.1625 103.632) (end 163.322 103.632) (width 0.25) (layer F.Cu) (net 5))
 (segment (start 156.845 102.7635) (end 153.7765 102.7635) (width 0.25) (layer F.Cu) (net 5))
 (segment (start 146.812 103.759) (end 144.587 101.534) (width 0.25) (layer F.Cu) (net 5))
 (segment (start 152.781 103.759) (end 146.812 103.759) (width 0.25) (layer F.Cu) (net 5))
 (segment (start 153.7765 102.7635) (end 152.781 103.759) (width 0.25) (layer F.Cu) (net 5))
 (segment (start 144.61 95.631) (end 144.61 93.134) (width 0.25) (layer F.Cu) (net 5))
 (segment (start 144.61 93.134) (end 144.907 92.837) (width 0.25) (layer F.Cu) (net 5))
 (segment (start 144.587 98.9965) (end 144.587 95.654) (width 0.25) (layer F.Cu) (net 5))
 (segment (start 144.587 95.654) (end 144.61 95.631) (width 0.25) (layer F.Cu) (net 5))
 (segment (start 140.335 106.68) (end 140.335 105.8545) (width 0.25) (layer F.Cu) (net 5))
 (segment (start 140.335 105.8545) (end 144.587 101.6025) (width 0.25) (layer F.Cu) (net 5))
 (segment (start 144.587 101.6025) (end 144.587 101.534) (width 0.25) (layer F.Cu) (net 5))
 (segment (start 144.587 101.534) (end 144.587 98.9965) (width 0.25) (layer F.Cu) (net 5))
 (segment (start 160.4215 95.758) (end 162.6845 95.758) (width 0.25) (layer F.Cu) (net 6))
 (segment (start 162.6845 95.758) (end 162.687 95.7555) (width 0.25) (layer F.Cu) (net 6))
 (segment (start 160.41905 98.20395) (end 160.41905 95.76045) (width 0.25) (layer F.Cu) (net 6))
 (segment (start 160.41905 95.76045) (end 160.2715 95.6129) (width 0.25) (layer F.Cu) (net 6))
 (segment (start 160.2715 95.6129) (end 160.2715 93.853) (width 0.25) (layer F.Cu) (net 6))
 (segment (start 156.845 100.5635) (end 156.845 98.222) (width 0.25) (layer F.Cu) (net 7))
 (segment (start 156.845 98.222) (end 156.82695 98.20395) (width 0.25) (layer F.Cu) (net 7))
 (segment (start 142.875 109.22) (end 163.627 109.22) (width 0.25) (layer F.Cu) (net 9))
 (segment (start 163.627 109.22) (end 165.4835 107.3635) (width 0.25) (layer F.Cu) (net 9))
 (segment (start 165.4835 104.8535) (end 150.8275 104.8535) (width 0.25) (layer F.Cu) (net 8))
 (segment (start 139.319 95.631) (end 142.41 95.631) (width 0.25) (layer F.Cu) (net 8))
 (via (at 139.319 95.631) (size 0.6) (drill 0.4) (layers F.Cu B.Cu) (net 8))
 (segment (start 139.319 101.4095) (end 139.319 95.631) (width 0.25) (layer B.Cu) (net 8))
 (segment (start 142.748 104.8385) (end 139.319 101.4095) (width 0.25) (layer B.Cu) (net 8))
 (segment (start 150.8125 104.8385) (end 142.748 104.8385) (width 0.25) (layer B.Cu) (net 8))
 (via (at 150.8125 104.8385) (size 0.6) (drill 0.4) (layers F.Cu B.Cu) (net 8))
 (segment (start 150.8275 104.8535) (end 150.8125 104.8385) (width 0.25) (layer F.Cu) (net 8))
 (segment (start 142.367 92.837) (end 142.367 95.588) (width 0.25) (layer F.Cu) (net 8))
 (segment (start 142.367 95.588) (end 142.41 95.631) (width 0.25) (layer F.Cu) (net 8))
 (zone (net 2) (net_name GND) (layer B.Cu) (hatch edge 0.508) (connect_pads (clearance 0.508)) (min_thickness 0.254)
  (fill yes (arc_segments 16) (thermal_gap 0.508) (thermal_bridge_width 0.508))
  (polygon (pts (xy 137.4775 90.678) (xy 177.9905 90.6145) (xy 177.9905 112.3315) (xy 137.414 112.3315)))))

